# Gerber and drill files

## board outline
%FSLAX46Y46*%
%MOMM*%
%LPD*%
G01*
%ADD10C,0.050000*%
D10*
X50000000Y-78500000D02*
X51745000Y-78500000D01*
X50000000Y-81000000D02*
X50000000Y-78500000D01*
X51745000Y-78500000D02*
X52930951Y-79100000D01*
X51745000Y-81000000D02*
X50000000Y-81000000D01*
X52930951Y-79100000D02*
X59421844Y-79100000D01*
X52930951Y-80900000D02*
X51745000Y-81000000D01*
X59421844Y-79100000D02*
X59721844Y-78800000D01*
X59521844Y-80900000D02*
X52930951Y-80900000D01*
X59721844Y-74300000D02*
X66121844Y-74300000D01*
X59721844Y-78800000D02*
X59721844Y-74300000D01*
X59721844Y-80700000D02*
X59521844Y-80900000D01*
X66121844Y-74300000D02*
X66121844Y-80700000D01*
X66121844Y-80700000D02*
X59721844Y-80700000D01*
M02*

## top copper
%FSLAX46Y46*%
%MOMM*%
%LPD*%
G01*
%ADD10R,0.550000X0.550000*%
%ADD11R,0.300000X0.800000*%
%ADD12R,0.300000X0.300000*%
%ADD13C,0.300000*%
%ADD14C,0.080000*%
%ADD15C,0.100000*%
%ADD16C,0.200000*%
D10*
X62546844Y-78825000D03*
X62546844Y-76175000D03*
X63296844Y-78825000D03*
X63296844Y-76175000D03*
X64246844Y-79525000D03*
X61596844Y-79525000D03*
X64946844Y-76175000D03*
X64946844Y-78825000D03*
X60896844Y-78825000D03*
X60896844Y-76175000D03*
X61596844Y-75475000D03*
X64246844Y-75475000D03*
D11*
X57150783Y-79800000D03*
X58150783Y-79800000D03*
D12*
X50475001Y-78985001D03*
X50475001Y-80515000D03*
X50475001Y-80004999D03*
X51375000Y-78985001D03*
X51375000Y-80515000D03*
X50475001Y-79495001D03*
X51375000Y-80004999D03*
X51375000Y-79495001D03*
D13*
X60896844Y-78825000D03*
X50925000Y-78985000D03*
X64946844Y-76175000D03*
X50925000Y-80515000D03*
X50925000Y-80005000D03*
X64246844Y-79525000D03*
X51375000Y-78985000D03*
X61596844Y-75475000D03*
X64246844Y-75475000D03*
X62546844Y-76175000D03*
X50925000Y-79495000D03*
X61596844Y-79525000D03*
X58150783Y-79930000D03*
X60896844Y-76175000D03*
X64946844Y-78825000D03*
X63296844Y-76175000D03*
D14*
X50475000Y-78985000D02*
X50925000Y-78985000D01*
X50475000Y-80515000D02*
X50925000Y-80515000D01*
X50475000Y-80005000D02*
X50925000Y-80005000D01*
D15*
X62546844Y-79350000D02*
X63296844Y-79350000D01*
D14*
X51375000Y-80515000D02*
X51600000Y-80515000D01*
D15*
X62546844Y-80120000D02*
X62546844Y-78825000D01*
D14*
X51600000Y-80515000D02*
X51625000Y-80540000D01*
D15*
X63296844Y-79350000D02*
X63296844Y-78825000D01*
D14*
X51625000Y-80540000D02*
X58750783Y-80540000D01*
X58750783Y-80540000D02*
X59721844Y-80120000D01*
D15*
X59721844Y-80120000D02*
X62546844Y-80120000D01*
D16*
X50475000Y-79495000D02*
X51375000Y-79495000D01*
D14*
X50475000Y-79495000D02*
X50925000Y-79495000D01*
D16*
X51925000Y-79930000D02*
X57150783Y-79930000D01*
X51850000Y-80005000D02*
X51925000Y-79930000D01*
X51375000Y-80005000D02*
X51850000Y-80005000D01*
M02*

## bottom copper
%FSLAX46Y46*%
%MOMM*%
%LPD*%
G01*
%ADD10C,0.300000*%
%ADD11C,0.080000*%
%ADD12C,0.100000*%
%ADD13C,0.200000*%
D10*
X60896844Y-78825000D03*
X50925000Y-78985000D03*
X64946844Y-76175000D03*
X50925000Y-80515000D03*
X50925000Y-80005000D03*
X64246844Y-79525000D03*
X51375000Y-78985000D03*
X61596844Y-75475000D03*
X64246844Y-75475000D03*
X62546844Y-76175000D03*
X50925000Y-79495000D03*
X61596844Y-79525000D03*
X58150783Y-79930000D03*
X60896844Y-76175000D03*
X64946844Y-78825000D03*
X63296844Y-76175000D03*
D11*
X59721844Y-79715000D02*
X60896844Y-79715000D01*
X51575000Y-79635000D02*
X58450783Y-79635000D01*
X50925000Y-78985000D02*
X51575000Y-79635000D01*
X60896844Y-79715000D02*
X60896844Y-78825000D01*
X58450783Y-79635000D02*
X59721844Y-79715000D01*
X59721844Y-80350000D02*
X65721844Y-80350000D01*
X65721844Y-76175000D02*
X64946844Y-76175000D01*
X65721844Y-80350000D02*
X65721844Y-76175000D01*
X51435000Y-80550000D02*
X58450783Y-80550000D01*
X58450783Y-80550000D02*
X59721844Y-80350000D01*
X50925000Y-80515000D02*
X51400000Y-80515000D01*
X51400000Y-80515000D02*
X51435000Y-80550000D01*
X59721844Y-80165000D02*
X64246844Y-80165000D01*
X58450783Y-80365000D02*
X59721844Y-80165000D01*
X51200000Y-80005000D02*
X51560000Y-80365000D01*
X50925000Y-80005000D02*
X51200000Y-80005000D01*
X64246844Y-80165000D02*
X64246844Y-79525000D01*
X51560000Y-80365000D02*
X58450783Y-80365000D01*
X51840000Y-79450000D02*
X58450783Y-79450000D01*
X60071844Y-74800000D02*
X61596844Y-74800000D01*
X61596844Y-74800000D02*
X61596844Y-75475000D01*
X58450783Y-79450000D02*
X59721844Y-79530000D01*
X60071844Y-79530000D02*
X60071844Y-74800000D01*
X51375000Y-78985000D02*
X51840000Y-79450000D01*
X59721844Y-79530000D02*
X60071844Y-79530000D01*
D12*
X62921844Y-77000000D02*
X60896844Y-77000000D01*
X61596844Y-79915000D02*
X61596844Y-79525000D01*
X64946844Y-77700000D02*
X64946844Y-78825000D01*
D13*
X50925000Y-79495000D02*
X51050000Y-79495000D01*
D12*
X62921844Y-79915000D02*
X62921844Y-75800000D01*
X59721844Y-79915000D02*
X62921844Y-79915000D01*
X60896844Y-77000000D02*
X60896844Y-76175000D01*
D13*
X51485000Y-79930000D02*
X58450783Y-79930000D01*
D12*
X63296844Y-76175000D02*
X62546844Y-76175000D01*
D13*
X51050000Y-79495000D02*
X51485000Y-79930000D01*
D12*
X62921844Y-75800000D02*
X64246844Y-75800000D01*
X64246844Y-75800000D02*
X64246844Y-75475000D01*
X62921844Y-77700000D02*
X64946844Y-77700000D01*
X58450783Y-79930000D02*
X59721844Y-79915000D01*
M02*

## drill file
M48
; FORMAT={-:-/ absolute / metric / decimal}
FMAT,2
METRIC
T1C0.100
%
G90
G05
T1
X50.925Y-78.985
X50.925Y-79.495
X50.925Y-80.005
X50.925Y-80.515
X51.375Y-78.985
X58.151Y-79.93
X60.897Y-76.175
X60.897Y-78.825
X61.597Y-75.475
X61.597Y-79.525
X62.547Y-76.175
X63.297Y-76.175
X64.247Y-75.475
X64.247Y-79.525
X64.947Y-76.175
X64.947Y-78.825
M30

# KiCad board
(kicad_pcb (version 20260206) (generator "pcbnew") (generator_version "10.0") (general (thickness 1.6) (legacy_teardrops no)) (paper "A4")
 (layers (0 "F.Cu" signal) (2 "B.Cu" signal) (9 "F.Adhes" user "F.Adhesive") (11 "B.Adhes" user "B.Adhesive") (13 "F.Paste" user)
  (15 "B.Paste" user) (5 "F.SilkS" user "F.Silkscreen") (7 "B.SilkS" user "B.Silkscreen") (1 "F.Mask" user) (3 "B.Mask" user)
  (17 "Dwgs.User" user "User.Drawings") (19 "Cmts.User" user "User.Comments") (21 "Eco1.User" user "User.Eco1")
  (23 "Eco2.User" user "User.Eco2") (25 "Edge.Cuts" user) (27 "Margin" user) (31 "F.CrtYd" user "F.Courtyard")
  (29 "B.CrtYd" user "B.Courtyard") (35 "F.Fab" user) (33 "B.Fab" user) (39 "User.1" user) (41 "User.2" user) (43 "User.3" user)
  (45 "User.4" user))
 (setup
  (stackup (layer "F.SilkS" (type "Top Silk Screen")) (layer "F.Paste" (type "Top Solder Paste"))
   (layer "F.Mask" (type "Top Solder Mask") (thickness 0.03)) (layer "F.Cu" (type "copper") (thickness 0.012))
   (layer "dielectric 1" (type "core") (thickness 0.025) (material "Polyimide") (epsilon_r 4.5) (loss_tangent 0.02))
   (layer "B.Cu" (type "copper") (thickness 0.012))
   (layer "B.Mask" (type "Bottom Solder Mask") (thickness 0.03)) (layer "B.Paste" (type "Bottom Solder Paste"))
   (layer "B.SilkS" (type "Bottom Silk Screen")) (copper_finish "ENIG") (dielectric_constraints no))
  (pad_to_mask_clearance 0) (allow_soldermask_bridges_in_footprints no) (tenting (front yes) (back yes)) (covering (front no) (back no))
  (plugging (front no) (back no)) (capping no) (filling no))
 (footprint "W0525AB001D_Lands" (layer "F.Cu") (at 57.650783 79.93)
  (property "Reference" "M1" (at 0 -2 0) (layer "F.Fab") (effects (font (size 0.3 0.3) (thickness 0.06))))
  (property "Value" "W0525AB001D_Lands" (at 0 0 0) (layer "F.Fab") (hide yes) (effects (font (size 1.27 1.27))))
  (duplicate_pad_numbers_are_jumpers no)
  (pad "1" smd rect (at -0.5 -0.13) (size 0.3 0.8) (layers "F.Cu" "F.Mask") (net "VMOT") (solder_mask_margin 0.05) (thermal_bridge_angle 45))
  (pad "2" smd rect (at 0.5 -0.13) (size 0.3 0.8) (layers "F.Cu" "F.Mask") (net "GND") (solder_mask_margin 0.05) (thermal_bridge_angle 45)))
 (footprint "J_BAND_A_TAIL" (layer "F.Cu") (at 50.9 79.75)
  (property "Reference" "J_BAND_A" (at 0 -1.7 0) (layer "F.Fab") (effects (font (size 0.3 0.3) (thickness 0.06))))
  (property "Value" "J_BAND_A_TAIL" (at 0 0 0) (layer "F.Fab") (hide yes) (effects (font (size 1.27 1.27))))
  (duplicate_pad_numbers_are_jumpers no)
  (pad "1" smd rect (at -0.424999 -0.764999) (size 0.3 0.3) (layers "F.Cu" "F.Mask") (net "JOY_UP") (solder_mask_margin 0.05)
   (thermal_bridge_angle 45))
  (pad "2" smd rect (at -0.424999 0.765) (size 0.3 0.3) (layers "F.Cu" "F.Mask") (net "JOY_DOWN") (solder_mask_margin 0.05)
   (thermal_bridge_angle 45))
  (pad "3" smd rect (at -0.424999 0.254999) (size 0.3 0.3) (layers "F.Cu" "F.Mask") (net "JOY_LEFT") (solder_mask_margin 0.05)
   (thermal_bridge_angle 45))
  (pad "4" smd rect (at 0.475 -0.764999) (size 0.3 0.3) (layers "F.Cu" "F.Mask") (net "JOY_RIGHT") (solder_mask_margin 0.05)
   (thermal_bridge_angle 45))
  (pad "5" smd rect (at 0.475 0.765) (size 0.3 0.3) (layers "F.Cu" "F.Mask") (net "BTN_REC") (solder_mask_margin 0.05)
   (thermal_bridge_angle 45))
  (pad "6" smd rect (at -0.424999 -0.254999) (size 0.3 0.3) (layers "F.Cu" "F.Mask") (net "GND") (solder_mask_margin 0.05)
   (thermal_bridge_angle 45))
  (pad "7" smd rect (at 0.475 0.254999) (size 0.3 0.3) (layers "F.Cu" "F.Mask") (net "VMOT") (solder_mask_margin 0.05)
   (thermal_bridge_angle 45))
  (pad "8" smd rect (at 0.475 -0.254999) (size 0.3 0.3) (layers "F.Cu" "F.Mask") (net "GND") (solder_mask_margin 0.05)
   (thermal_bridge_angle 45)))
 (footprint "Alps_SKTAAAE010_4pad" (layer "F.Cu") (at 62.921844 77.5 90)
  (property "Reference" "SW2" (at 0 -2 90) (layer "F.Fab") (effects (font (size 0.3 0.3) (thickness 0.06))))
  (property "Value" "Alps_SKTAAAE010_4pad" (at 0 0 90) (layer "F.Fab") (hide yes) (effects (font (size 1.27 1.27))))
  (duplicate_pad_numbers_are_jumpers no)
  (pad "1" smd rect (at -1.325 -0.375 90) (size 0.55 0.55) (layers "F.Cu" "F.Mask" "F.Paste") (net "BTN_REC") (solder_mask_margin 0.05)
   (thermal_bridge_angle 45))
  (pad "2" smd rect (at 1.325 -0.375 90) (size 0.55 0.55) (layers "F.Cu" "F.Mask" "F.Paste") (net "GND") (solder_mask_margin 0.05)
   (thermal_bridge_angle 45))
  (pad "3" smd rect (at -1.325 0.375 90) (size 0.55 0.55) (layers "F.Cu" "F.Mask" "F.Paste") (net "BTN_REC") (solder_mask_margin 0.05)
   (thermal_bridge_angle 45))
  (pad "4" smd rect (at 1.325 0.375 90) (size 0.55 0.55) (layers "F.Cu" "F.Mask" "F.Paste") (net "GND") (solder_mask_margin 0.05)
   (thermal_bridge_angle 45)))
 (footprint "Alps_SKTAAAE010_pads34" (layer "F.Cu") (at 62.921844 75.1)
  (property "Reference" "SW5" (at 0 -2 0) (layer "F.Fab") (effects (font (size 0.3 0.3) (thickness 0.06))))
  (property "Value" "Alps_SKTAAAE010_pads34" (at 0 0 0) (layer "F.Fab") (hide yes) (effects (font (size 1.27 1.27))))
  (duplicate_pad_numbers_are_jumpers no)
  (pad "3" smd rect (at -1.325 0.375) (size 0.55 0.55) (layers "F.Cu" "F.Mask" "F.Paste") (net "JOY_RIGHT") (solder_mask_margin 0.05)
   (thermal_bridge_angle 45))
  (pad "4" smd rect (at 1.325 0.375) (size 0.55 0.55) (layers "F.Cu" "F.Mask" "F.Paste") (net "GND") (solder_mask_margin 0.05)
   (thermal_bridge_angle 45)))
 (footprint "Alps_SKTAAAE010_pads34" (layer "F.Cu") (at 65.321844 77.5 -90)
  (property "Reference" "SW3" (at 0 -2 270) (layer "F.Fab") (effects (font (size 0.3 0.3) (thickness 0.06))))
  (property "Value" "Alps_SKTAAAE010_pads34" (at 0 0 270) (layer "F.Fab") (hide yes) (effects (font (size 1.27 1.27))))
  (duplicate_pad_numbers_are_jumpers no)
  (pad "3" smd rect (at -1.325 0.375 270) (size 0.55 0.55) (layers "F.Cu" "F.Mask" "F.Paste") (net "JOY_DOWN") (solder_mask_margin 0.05)
   (thermal_bridge_angle 45))
  (pad "4" smd rect (at 1.325 0.375 270) (size 0.55 0.55) (layers "F.Cu" "F.Mask" "F.Paste") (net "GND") (solder_mask_margin 0.05)
   (thermal_bridge_angle 45)))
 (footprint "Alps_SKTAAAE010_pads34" (layer "F.Cu") (at 62.921844 79.9 180)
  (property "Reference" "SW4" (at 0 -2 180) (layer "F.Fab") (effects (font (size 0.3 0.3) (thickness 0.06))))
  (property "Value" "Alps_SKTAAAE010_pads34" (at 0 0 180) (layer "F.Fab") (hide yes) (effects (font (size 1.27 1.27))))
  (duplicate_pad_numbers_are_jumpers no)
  (pad "3" smd rect (at -1.325 0.375 180) (size 0.55 0.55) (layers "F.Cu" "F.Mask" "F.Paste") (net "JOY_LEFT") (solder_mask_margin 0.05)
   (thermal_bridge_angle 45))
  (pad "4" smd rect (at 1.325 0.375 180) (size 0.55 0.55) (layers "F.Cu" "F.Mask" "F.Paste") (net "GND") (solder_mask_margin 0.05)
   (thermal_bridge_angle 45)))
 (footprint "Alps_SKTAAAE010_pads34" (layer "F.Cu") (at 60.521844 77.5 90)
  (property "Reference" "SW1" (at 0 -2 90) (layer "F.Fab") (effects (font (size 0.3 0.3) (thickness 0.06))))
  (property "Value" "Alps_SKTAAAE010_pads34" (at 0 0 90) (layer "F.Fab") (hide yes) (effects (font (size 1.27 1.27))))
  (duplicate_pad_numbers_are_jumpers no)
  (pad "3" smd rect (at -1.325 0.375 90) (size 0.55 0.55) (layers "F.Cu" "F.Mask" "F.Paste") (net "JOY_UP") (solder_mask_margin 0.05)
   (thermal_bridge_angle 45))
  (pad "4" smd rect (at 1.325 0.375 90) (size 0.55 0.55) (layers "F.Cu" "F.Mask" "F.Paste") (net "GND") (solder_mask_margin 0.05)
   (thermal_bridge_angle 45)))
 (gr_line (start 50 78.5) (end 51.745 78.5) (stroke (width 0.05) (type default)) (layer "Edge.Cuts"))
 (gr_line (start 50 81) (end 50 78.5) (stroke (width 0.05) (type default)) (layer "Edge.Cuts"))
 (gr_line (start 51.745 78.5) (end 52.930951 79.1) (stroke (width 0.05) (type default)) (layer "Edge.Cuts"))
 (gr_line (start 51.745 81) (end 50 81) (stroke (width 0.05) (type default)) (layer "Edge.Cuts"))
 (gr_line (start 52.930951 79.1) (end 59.421844 79.1) (stroke (width 0.05) (type default)) (layer "Edge.Cuts"))
 (gr_line (start 52.930951 80.9) (end 51.745 81) (stroke (width 0.05) (type default)) (layer "Edge.Cuts"))
 (gr_line (start 59.421844 79.1) (end 59.721844 78.8) (stroke (width 0.05) (type default)) (layer "Edge.Cuts"))
 (gr_line (start 59.521844 80.9) (end 52.930951 80.9) (stroke (width 0.05) (type default)) (layer "Edge.Cuts"))
 (gr_line (start 59.721844 74.3) (end 66.121844 74.3) (stroke (width 0.05) (type default)) (layer "Edge.Cuts"))
 (gr_line (start 59.721844 78.8) (end 59.721844 74.3) (stroke (width 0.05) (type default)) (layer "Edge.Cuts"))
 (gr_line (start 59.721844 80.7) (end 59.521844 80.9) (stroke (width 0.05) (type default)) (layer "Edge.Cuts"))
 (gr_line (start 66.121844 74.3) (end 66.121844 80.7) (stroke (width 0.05) (type default)) (layer "Edge.Cuts"))
 (gr_line (start 66.121844 80.7) (end 59.721844 80.7) (stroke (width 0.05) (type default)) (layer "Edge.Cuts"))
 (segment (start 51.925 79.93) (end 57.150783 79.93) (width 0.2) (layer "F.Cu") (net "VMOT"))
 (segment (start 51.85 80.005) (end 51.925 79.93) (width 0.2) (layer "F.Cu") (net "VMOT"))
 (segment (start 51.375 80.005) (end 51.85 80.005) (width 0.2) (layer "F.Cu") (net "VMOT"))
 (segment (start 50.475 79.495) (end 50.925 79.495) (width 0.08) (layer "F.Cu") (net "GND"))
 (segment (start 50.475 79.495) (end 51.375 79.495) (width 0.2) (layer "F.Cu") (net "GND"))
 (via (at 63.296844 76.175) (size 0.3) (drill 0.1) (layers "F.Cu" "B.Cu") (tenting (front yes) (back yes)) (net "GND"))
 (via (at 62.546844 76.175) (size 0.3) (drill 0.1) (layers "F.Cu" "B.Cu") (tenting (front yes) (back yes)) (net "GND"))
 (via (at 58.150783 79.93) (size 0.3) (drill 0.1) (layers "F.Cu" "B.Cu") (tenting (front yes) (back yes)) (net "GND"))
 (via (at 60.896844 76.175) (size 0.3) (drill 0.1) (layers "F.Cu" "B.Cu") (tenting (front yes) (back yes)) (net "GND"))
 (via (at 64.946844 78.825) (size 0.3) (drill 0.1) (layers "F.Cu" "B.Cu") (tenting (front yes) (back yes)) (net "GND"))
 (via (at 64.246844 75.475) (size 0.3) (drill 0.1) (layers "F.Cu" "B.Cu") (tenting (front yes) (back yes)) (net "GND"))
 (via (at 50.925 79.495) (size 0.3) (drill 0.1) (layers "F.Cu" "B.Cu") (tenting (front yes) (back yes)) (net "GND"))
 (via (at 61.596844 79.525) (size 0.3) (drill 0.1) (layers "F.Cu" "B.Cu") (tenting (front yes) (back yes)) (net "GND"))
 (segment (start 64.946844 77.7) (end 64.946844 78.825) (width 0.1) (layer "B.Cu") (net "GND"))
 (segment (start 64.246844 75.8) (end 64.246844 75.475) (width 0.1) (layer "B.Cu") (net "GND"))
 (segment (start 51.485 79.93) (end 58.450783 79.93) (width 0.2) (layer "B.Cu") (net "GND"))
 (segment (start 58.450783 79.93) (end 59.721844 79.915) (width 0.1) (layer "B.Cu") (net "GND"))
 (segment (start 59.721844 79.915) (end 62.921844 79.915) (width 0.1) (layer "B.Cu") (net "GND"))
 (segment (start 62.921844 75.8) (end 64.246844 75.8) (width 0.1) (layer "B.Cu") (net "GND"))
 (segment (start 50.925 79.495) (end 51.05 79.495) (width 0.2) (layer "B.Cu") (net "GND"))
 (segment (start 51.05 79.495) (end 51.485 79.93) (width 0.2) (layer "B.Cu") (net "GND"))
 (segment (start 62.921844 77.7) (end 64.946844 77.7) (width 0.1) (layer "B.Cu") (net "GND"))
 (segment (start 61.596844 79.915) (end 61.596844 79.525) (width 0.1) (layer "B.Cu") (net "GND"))
 (segment (start 63.296844 76.175) (end 62.546844 76.175) (width 0.1) (layer "B.Cu") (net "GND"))
 (segment (start 60.896844 77) (end 60.896844 76.175) (width 0.1) (layer "B.Cu") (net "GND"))
 (segment (start 62.921844 77) (end 60.896844 77) (width 0.1) (layer "B.Cu") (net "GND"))
 (segment (start 62.921844 79.915) (end 62.921844 75.8) (width 0.1) (layer "B.Cu") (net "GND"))
 (segment (start 50.475 78.985) (end 50.925 78.985) (width 0.08) (layer "F.Cu") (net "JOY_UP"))
 (via (at 60.896844 78.825) (size 0.3) (drill 0.1) (layers "F.Cu" "B.Cu") (tenting (front yes) (back yes)) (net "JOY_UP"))
 (via (at 50.925 78.985) (size 0.3) (drill 0.1) (layers "F.Cu" "B.Cu") (tenting (front yes) (back yes)) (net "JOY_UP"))
 (segment (start 51.575 79.635) (end 58.450783 79.635) (width 0.08) (layer "B.Cu") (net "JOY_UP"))
 (segment (start 60.896844 79.715) (end 60.896844 78.825) (width 0.08) (layer "B.Cu") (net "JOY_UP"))
 (segment (start 59.721844 79.715) (end 60.896844 79.715) (width 0.08) (layer "B.Cu") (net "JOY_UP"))
 (segment (start 50.925 78.985) (end 51.575 79.635) (width 0.08) (layer "B.Cu") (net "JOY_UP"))
 (segment (start 58.450783 79.635) (end 59.721844 79.715) (width 0.08) (layer "B.Cu") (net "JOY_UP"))
 (segment (start 50.475 80.515) (end 50.925 80.515) (width 0.08) (layer "F.Cu") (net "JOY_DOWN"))
 (via (at 50.925 80.515) (size 0.3) (drill 0.1) (layers "F.Cu" "B.Cu") (tenting (front yes) (back yes)) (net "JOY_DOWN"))
 (via (at 64.946844 76.175) (size 0.3) (drill 0.1) (layers "F.Cu" "B.Cu") (tenting (front yes) (back yes)) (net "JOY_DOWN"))
 (segment (start 59.721844 80.35) (end 65.721844 80.35) (width 0.08) (layer "B.Cu") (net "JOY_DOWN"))
 (segment (start 65.721844 80.35) (end 65.721844 76.175) (width 0.08) (layer "B.Cu") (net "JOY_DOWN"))
 (segment (start 51.4 80.515) (end 51.435 80.55) (width 0.08) (layer "B.Cu") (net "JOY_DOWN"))
 (segment (start 65.721844 76.175) (end 64.946844 76.175) (width 0.08) (layer "B.Cu") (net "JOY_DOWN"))
 (segment (start 50.925 80.515) (end 51.4 80.515) (width 0.08) (layer "B.Cu") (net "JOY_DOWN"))
 (segment (start 58.450783 80.55) (end 59.721844 80.35) (width 0.08) (layer "B.Cu") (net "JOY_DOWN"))
 (segment (start 51.435 80.55) (end 58.450783 80.55) (width 0.08) (layer "B.Cu") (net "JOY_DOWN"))
 (segment (start 50.475 80.005) (end 50.925 80.005) (width 0.08) (layer "F.Cu") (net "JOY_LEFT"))
 (via (at 50.925 80.005) (size 0.3) (drill 0.1) (layers "F.Cu" "B.Cu") (tenting (front yes) (back yes)) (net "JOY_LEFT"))
 (via (at 64.246844 79.525) (size 0.3) (drill 0.1) (layers "F.Cu" "B.Cu") (tenting (front yes) (back yes)) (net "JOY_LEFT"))
 (segment (start 51.2 80.005) (end 51.56 80.365) (width 0.08) (layer "B.Cu") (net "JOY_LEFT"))
 (segment (start 51.56 80.365) (end 58.450783 80.365) (width 0.08) (layer "B.Cu") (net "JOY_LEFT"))
 (segment (start 59.721844 80.165) (end 64.246844 80.165) (width 0.08) (layer "B.Cu") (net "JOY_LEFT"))
 (segment (start 50.925 80.005) (end 51.2 80.005) (width 0.08) (layer "B.Cu") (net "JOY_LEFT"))
 (segment (start 58.450783 80.365) (end 59.721844 80.165) (width 0.08) (layer "B.Cu") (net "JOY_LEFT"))
 (segment (start 64.246844 80.165) (end 64.246844 79.525) (width 0.08) (layer "B.Cu") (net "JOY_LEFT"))
 (via (at 61.596844 75.475) (size 0.3) (drill 0.1) (layers "F.Cu" "B.Cu") (tenting (front yes) (back yes)) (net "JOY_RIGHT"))
 (via (at 51.375 78.985) (size 0.3) (drill 0.1) (layers "F.Cu" "B.Cu") (tenting (front yes) (back yes)) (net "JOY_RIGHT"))
 (segment (start 60.071844 79.53) (end 60.071844 74.8) (width 0.08) (layer "B.Cu") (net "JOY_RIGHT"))
 (segment (start 58.450783 79.45) (end 59.721844 79.53) (width 0.08) (layer "B.Cu") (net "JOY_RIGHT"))
 (segment (start 59.721844 79.53) (end 60.071844 79.53) (width 0.08) (layer "B.Cu") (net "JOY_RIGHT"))
 (segment (start 51.84 79.45) (end 58.450783 79.45) (width 0.08) (layer "B.Cu") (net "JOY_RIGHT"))
 (segment (start 60.071844 74.8) (end 61.596844 74.8) (width 0.08) (layer "B.Cu") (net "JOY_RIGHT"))
 (segment (start 61.596844 74.8) (end 61.596844 75.475) (width 0.08) (layer "B.Cu") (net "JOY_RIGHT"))
 (segment (start 51.375 78.985) (end 51.84 79.45) (width 0.08) (layer "B.Cu") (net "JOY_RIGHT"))
 (segment (start 62.546844 79.35) (end 63.296844 79.35) (width 0.1) (layer "F.Cu") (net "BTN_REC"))
 (segment (start 62.546844 80.12) (end 62.546844 78.825) (width 0.1) (layer "F.Cu") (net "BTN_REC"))
 (segment (start 51.625 80.54) (end 58.750783 80.54) (width 0.08) (layer "F.Cu") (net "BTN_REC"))
 (segment (start 59.721844 80.12) (end 62.546844 80.12) (width 0.1) (layer "F.Cu") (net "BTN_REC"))
 (segment (start 58.750783 80.54) (end 59.721844 80.12) (width 0.08) (layer "F.Cu") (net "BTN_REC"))
 (segment (start 51.6 80.515) (end 51.625 80.54) (width 0.08) (layer "F.Cu") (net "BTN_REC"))
 (segment (start 63.296844 79.35) (end 63.296844 78.825) (width 0.1) (layer "F.Cu") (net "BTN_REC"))
 (segment (start 51.375 80.515) (end 51.6 80.515) (width 0.08) (layer "F.Cu") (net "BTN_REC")))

